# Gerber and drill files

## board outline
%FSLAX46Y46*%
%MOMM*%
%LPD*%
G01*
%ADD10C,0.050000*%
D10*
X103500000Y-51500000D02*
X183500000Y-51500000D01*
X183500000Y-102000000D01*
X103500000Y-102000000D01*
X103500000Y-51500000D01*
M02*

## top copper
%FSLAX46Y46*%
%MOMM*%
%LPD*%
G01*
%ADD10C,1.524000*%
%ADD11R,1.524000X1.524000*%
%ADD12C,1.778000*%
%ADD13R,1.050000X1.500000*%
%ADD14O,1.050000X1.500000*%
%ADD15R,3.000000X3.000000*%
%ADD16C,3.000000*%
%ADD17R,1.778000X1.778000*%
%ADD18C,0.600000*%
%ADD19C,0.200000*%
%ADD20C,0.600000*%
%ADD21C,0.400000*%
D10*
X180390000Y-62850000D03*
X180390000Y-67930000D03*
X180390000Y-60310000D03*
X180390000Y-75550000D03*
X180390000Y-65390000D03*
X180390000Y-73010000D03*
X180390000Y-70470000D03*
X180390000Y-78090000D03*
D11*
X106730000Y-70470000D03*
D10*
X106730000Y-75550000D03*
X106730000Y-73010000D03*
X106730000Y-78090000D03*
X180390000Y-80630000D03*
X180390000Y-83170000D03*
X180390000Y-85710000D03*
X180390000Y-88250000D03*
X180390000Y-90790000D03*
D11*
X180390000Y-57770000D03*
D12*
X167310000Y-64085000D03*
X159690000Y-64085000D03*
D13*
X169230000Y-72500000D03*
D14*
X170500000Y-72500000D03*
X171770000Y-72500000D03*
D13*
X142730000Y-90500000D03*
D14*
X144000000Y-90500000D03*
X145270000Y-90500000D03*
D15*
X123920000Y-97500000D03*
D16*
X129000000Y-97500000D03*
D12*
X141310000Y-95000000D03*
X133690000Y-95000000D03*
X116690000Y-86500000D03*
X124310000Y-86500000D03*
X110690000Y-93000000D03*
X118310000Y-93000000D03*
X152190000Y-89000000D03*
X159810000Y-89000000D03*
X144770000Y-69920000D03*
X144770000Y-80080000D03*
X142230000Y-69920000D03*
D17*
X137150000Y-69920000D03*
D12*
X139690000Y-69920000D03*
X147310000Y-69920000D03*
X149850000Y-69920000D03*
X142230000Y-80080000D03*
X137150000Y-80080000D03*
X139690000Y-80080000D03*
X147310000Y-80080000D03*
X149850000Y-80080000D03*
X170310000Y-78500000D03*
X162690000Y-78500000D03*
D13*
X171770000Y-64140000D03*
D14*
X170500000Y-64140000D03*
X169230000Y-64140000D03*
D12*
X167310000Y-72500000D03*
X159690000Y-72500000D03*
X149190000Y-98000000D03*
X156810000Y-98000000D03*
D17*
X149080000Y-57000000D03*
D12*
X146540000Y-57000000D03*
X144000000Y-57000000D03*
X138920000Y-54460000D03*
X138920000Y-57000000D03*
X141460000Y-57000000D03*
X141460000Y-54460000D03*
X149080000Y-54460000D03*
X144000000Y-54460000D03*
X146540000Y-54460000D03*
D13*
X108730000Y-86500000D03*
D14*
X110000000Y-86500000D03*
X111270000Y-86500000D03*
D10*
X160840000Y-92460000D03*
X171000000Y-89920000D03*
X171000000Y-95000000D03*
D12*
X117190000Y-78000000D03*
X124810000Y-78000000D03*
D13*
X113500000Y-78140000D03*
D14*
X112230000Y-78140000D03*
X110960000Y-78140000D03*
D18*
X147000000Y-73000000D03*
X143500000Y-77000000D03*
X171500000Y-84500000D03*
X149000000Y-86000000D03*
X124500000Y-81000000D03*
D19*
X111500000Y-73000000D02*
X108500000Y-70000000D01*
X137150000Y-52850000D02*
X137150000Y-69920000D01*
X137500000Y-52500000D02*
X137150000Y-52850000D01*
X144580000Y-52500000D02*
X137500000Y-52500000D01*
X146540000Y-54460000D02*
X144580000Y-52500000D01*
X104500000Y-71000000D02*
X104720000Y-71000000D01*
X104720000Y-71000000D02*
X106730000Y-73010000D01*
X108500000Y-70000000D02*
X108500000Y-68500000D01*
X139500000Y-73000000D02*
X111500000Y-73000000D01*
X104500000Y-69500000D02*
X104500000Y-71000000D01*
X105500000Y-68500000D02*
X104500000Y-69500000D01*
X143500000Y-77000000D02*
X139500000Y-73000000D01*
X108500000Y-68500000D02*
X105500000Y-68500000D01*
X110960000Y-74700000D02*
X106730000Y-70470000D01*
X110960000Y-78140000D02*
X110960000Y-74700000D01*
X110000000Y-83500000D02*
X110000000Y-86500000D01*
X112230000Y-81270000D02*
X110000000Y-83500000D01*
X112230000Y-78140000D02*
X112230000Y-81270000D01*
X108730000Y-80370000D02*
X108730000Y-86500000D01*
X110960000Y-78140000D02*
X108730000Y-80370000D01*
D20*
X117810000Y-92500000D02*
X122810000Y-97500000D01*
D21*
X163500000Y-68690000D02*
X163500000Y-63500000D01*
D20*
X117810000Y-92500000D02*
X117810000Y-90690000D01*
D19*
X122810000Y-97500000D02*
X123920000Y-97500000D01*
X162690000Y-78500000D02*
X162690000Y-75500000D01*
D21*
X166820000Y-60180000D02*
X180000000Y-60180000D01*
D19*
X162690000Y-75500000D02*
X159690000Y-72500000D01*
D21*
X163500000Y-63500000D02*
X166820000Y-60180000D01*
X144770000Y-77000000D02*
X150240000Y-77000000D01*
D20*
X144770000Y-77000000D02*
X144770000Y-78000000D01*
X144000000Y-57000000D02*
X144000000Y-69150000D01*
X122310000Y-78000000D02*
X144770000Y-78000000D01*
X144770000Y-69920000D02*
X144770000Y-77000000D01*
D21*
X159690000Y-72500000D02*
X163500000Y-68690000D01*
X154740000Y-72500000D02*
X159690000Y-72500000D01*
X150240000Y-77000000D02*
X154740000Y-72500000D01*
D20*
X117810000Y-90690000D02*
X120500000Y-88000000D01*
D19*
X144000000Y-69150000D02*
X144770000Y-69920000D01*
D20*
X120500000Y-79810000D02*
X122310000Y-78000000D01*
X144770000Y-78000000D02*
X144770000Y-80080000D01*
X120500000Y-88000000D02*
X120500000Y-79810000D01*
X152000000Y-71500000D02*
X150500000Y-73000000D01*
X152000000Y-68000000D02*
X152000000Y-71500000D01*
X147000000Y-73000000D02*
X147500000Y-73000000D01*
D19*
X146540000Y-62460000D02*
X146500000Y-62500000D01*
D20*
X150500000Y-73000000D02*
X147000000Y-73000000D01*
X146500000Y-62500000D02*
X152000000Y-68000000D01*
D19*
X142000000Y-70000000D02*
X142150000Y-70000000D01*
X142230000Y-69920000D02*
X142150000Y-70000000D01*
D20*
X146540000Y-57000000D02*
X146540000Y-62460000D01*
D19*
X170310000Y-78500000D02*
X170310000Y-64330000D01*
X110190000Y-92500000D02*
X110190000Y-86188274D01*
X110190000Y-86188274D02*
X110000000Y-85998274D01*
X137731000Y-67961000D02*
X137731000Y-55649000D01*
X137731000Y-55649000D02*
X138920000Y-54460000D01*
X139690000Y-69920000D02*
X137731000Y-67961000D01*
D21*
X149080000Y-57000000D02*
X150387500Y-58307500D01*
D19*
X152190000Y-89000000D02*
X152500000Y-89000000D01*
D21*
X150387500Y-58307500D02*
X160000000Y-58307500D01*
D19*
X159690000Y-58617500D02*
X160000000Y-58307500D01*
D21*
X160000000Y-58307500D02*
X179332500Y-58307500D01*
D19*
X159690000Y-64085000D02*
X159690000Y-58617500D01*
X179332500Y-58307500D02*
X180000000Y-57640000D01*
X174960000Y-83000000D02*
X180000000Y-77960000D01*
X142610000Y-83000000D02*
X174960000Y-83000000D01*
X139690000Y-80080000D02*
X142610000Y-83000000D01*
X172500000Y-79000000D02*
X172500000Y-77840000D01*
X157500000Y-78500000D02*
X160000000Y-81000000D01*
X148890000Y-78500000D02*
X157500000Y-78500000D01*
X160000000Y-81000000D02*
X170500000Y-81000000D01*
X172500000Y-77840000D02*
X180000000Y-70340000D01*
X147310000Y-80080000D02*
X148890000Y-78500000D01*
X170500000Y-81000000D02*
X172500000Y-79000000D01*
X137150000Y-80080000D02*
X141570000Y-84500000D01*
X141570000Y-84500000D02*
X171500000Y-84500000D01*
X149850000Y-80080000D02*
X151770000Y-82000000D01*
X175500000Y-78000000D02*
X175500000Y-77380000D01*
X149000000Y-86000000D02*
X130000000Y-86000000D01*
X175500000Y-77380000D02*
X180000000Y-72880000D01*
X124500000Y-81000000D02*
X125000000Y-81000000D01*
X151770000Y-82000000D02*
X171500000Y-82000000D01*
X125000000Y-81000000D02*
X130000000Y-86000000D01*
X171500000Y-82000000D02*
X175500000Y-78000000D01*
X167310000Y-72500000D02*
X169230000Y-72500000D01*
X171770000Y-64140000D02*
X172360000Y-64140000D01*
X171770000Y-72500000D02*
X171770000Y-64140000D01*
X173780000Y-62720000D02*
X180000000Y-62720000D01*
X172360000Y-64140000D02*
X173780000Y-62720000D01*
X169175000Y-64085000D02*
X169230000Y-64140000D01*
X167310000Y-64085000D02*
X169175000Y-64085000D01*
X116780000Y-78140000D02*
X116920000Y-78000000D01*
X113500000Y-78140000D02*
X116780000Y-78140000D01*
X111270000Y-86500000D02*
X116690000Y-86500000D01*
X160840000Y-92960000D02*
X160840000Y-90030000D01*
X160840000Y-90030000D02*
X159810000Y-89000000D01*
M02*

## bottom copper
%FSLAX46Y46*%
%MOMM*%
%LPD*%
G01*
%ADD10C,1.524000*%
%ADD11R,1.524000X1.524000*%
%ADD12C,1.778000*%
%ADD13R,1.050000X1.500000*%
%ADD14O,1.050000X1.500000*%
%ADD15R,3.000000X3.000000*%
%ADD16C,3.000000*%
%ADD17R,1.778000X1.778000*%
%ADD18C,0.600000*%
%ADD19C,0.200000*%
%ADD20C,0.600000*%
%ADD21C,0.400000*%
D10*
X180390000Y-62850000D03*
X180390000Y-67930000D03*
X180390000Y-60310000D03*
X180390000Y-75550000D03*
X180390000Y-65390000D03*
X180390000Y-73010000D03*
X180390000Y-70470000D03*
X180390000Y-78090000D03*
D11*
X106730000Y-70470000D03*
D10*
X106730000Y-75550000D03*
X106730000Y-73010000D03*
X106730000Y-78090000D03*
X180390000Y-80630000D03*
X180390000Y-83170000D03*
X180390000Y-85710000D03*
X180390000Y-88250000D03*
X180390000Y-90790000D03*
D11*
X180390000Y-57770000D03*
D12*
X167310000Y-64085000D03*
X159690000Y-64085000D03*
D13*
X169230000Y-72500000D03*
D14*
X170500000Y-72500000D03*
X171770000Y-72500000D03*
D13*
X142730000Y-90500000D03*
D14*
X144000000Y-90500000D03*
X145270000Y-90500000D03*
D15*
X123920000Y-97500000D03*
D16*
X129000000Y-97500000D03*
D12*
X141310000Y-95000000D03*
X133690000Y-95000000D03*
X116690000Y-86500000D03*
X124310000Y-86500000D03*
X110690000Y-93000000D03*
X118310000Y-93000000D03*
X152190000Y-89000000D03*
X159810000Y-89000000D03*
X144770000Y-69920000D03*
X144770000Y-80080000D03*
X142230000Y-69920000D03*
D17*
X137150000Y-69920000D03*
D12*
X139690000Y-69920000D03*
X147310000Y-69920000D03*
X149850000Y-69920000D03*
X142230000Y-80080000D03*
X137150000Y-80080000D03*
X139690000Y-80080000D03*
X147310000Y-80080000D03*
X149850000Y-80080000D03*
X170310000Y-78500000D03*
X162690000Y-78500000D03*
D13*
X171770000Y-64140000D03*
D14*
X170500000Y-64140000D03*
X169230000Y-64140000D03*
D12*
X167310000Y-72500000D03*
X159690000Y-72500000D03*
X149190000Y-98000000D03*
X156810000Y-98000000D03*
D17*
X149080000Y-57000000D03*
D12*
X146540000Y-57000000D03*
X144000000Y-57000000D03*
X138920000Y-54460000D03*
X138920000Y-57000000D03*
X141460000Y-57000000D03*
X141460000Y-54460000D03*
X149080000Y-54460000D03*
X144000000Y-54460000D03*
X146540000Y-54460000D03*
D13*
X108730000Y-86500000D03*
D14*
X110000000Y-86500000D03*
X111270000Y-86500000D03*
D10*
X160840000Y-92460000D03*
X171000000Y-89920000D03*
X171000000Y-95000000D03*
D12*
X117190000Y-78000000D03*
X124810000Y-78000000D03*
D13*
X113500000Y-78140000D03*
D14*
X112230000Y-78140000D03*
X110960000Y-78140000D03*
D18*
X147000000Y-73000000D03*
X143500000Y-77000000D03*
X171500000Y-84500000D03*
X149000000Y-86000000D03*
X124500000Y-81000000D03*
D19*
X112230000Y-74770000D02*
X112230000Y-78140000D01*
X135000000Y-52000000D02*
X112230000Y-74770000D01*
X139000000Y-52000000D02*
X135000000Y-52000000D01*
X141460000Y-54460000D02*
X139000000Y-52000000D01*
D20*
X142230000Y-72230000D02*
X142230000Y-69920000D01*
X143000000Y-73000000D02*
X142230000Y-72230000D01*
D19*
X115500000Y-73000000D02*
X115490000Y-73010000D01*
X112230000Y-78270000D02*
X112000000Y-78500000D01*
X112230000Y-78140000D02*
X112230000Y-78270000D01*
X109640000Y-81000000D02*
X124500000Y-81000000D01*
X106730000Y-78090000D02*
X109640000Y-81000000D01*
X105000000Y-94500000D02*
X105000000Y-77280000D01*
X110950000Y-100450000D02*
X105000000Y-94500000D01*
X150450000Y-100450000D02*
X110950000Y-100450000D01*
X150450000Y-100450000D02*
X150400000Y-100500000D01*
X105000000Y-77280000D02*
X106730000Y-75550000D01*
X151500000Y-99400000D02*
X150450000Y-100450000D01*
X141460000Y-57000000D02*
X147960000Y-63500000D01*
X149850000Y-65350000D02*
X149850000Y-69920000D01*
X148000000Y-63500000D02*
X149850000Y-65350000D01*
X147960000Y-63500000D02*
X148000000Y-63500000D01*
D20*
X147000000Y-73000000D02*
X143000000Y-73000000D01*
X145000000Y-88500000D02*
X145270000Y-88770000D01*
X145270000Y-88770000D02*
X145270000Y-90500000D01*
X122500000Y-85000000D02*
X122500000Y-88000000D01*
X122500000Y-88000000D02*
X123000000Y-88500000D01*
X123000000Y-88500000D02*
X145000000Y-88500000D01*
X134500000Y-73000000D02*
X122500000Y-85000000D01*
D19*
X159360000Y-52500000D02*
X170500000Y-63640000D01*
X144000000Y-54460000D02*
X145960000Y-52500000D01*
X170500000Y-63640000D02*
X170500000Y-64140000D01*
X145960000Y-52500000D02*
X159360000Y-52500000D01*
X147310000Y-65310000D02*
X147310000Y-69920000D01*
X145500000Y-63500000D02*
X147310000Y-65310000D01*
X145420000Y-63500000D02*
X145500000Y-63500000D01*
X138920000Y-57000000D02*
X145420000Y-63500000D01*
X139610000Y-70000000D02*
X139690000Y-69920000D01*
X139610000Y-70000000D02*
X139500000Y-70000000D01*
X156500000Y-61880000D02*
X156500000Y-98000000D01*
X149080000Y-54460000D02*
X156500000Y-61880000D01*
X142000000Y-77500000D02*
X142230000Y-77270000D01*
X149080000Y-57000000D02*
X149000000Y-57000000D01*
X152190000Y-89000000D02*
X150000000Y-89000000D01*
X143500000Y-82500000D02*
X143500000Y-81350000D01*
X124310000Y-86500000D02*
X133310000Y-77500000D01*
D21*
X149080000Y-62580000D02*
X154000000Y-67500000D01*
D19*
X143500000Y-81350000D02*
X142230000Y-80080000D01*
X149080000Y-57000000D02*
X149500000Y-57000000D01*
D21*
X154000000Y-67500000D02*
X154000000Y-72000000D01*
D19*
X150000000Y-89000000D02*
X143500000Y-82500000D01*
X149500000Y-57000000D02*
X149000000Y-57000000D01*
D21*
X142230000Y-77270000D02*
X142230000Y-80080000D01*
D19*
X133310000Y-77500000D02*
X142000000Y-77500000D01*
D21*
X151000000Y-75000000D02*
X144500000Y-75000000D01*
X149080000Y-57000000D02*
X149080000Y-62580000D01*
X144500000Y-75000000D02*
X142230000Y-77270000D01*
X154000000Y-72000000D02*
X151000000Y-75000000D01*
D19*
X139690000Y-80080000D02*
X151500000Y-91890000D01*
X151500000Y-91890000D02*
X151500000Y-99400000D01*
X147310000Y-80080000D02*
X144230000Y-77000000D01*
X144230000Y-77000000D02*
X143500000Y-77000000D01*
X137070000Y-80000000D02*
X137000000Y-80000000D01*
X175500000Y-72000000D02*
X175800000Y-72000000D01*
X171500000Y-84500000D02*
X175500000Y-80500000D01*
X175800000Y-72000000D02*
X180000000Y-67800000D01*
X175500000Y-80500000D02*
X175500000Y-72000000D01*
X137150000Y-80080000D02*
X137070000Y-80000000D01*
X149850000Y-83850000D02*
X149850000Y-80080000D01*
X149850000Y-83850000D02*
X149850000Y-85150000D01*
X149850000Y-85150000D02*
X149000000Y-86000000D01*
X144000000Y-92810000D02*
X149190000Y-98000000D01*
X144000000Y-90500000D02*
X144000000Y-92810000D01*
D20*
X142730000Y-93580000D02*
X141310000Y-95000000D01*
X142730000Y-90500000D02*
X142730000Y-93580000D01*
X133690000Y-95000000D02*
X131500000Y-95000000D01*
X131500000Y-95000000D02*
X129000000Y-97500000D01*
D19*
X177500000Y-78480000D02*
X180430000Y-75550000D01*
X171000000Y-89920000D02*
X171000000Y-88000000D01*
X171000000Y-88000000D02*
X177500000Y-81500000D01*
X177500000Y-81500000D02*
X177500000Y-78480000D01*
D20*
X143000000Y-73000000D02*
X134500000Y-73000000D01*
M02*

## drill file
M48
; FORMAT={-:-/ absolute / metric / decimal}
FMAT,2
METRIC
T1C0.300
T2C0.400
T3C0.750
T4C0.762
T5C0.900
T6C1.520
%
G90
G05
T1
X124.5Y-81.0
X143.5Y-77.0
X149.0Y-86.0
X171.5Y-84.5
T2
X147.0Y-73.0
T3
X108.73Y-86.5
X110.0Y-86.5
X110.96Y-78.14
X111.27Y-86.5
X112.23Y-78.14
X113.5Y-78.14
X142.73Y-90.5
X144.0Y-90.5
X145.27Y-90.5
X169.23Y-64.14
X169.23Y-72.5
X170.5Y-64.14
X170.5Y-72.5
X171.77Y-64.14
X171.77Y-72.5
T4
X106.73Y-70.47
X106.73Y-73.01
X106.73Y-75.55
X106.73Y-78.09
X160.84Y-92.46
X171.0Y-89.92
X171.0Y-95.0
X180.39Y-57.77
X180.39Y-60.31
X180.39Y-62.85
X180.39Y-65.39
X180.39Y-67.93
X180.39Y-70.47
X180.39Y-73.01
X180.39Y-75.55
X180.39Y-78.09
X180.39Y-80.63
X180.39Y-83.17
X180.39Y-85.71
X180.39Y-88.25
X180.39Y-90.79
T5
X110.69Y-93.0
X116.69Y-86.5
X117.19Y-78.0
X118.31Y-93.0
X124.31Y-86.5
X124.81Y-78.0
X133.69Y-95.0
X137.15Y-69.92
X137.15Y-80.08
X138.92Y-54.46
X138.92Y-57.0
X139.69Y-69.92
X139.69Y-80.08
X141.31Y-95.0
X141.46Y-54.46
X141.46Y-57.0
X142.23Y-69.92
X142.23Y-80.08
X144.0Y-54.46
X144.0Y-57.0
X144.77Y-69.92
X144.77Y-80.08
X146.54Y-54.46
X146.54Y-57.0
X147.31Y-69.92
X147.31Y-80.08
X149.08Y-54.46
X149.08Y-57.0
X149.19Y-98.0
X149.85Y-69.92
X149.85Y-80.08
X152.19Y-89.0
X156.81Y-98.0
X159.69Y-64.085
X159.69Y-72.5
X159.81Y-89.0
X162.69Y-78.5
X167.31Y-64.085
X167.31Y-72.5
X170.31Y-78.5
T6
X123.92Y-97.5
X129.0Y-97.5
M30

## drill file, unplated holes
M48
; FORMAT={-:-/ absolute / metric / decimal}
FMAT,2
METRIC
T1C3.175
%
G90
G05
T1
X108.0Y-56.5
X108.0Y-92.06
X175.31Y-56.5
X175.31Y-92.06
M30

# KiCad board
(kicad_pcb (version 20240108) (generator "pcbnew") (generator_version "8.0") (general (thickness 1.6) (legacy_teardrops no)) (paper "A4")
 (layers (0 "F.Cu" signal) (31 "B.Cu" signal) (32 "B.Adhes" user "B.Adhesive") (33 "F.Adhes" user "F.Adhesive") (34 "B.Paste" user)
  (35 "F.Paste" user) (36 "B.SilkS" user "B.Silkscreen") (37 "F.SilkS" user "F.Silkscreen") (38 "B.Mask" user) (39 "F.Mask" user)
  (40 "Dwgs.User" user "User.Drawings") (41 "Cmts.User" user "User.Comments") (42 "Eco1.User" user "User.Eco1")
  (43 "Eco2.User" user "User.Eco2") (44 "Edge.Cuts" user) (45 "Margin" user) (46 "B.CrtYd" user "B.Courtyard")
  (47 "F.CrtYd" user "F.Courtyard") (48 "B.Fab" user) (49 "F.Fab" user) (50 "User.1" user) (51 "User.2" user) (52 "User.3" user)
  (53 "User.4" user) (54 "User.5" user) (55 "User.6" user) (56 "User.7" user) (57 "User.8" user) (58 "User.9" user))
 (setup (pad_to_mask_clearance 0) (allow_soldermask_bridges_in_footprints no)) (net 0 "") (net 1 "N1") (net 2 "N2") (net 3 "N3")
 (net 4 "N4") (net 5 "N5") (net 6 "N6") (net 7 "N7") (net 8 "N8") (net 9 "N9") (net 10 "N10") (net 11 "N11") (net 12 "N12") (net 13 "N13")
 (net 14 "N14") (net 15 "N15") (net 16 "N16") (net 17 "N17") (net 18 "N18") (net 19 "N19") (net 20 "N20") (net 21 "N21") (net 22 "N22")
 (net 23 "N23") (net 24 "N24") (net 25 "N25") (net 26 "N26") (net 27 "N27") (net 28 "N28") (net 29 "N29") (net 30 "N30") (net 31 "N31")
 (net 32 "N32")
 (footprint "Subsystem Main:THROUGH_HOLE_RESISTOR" (layer "F.Cu") (at 163.5 64.085 180)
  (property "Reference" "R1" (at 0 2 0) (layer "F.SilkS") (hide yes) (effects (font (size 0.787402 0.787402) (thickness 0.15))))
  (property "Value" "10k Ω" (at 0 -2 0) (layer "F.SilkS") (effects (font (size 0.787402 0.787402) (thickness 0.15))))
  (pad "P$1" thru_hole circle (at -3.81 0 180) (size 1.778 1.778) (drill 0.9) (layers "*.Cu" "*.Mask") (remove_unused_layers no)
   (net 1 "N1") (solder_mask_margin 0.102))
  (pad "P$2" thru_hole circle (at 3.81 0 180) (size 1.778 1.778) (drill 0.9) (layers "*.Cu" "*.Mask") (remove_unused_layers no) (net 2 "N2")
   (solder_mask_margin 0.102)))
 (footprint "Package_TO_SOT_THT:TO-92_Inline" (layer "F.Cu") (at 169.23 72.5)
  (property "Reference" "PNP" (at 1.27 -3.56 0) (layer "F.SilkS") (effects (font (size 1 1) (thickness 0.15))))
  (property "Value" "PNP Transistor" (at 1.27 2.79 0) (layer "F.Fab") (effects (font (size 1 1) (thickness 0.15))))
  (pad "1" thru_hole rect (at 0 0) (size 1.05 1.5) (drill 0.75) (layers "*.Cu" "*.Mask") (remove_unused_layers no) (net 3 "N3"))
  (pad "2" thru_hole oval (at 1.27 0) (size 1.05 1.5) (drill 0.75) (layers "*.Cu" "*.Mask") (remove_unused_layers no) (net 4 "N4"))
  (pad "3" thru_hole oval (at 2.54 0) (size 1.05 1.5) (drill 0.75) (layers "*.Cu" "*.Mask") (remove_unused_layers no) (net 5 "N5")))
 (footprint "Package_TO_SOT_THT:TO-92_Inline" (layer "F.Cu") (at 142.73 90.5)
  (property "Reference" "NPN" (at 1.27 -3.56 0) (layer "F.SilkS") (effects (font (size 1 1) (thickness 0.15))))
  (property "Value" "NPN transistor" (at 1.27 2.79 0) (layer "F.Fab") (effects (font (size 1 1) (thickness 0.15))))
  (pad "1" thru_hole rect (at 0 0) (size 1.05 1.5) (drill 0.75) (layers "*.Cu" "*.Mask") (remove_unused_layers no) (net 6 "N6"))
  (pad "2" thru_hole oval (at 1.27 0) (size 1.05 1.5) (drill 0.75) (layers "*.Cu" "*.Mask") (remove_unused_layers no) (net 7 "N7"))
  (pad "3" thru_hole oval (at 2.54 0) (size 1.05 1.5) (drill 0.75) (layers "*.Cu" "*.Mask") (remove_unused_layers no) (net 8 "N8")))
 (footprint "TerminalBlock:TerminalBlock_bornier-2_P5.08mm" (layer "F.Cu") (at 123.92 97.5)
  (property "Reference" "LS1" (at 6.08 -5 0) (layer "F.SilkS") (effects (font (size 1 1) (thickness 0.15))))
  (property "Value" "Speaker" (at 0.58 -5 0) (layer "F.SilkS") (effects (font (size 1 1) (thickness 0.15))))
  (pad "1" thru_hole rect (at 0 0) (size 3 3) (drill 1.52) (layers "*.Cu" "*.Mask") (remove_unused_layers no) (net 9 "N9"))
  (pad "2" thru_hole circle (at 5.08 0) (size 3 3) (drill 1.52) (layers "*.Cu" "*.Mask") (remove_unused_layers no) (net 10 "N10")))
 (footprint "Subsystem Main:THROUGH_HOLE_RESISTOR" (layer "F.Cu") (at 137.5 95 180)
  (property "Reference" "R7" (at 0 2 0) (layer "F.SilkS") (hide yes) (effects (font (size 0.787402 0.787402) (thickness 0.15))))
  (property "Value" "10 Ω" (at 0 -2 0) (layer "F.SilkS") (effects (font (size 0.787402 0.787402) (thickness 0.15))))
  (pad "P$1" thru_hole circle (at -3.81 0 180) (size 1.778 1.778) (drill 0.9) (layers "*.Cu" "*.Mask") (remove_unused_layers no)
   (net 6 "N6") (solder_mask_margin 0.102))
  (pad "P$2" thru_hole circle (at 3.81 0 180) (size 1.778 1.778) (drill 0.9) (layers "*.Cu" "*.Mask") (remove_unused_layers no)
   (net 10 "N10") (solder_mask_margin 0.102)))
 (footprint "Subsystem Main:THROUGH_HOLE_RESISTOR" (layer "F.Cu") (at 120.5 86.5)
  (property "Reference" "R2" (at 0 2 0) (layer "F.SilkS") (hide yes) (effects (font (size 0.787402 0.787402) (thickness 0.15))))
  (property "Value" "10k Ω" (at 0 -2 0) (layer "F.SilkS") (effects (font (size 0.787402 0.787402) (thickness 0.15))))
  (pad "P$1" thru_hole circle (at -3.81 0) (size 1.778 1.778) (drill 0.9) (layers "*.Cu" "*.Mask") (remove_unused_layers no) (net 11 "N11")
   (solder_mask_margin 0.102))
  (pad "P$2" thru_hole circle (at 3.81 0) (size 1.778 1.778) (drill 0.9) (layers "*.Cu" "*.Mask") (remove_unused_layers no) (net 2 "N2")
   (solder_mask_margin 0.102)))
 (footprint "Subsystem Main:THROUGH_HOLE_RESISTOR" (layer "F.Cu") (at 114.5 93)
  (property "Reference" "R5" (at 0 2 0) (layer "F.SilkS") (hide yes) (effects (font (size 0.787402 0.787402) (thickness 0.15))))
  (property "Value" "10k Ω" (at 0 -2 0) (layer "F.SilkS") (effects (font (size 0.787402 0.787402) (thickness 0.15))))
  (pad "P$1" thru_hole circle (at -3.81 0) (size 1.778 1.778) (drill 0.9) (layers "*.Cu" "*.Mask") (remove_unused_layers no) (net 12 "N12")
   (solder_mask_margin 0.102))
  (pad "P$2" thru_hole circle (at 3.81 0) (size 1.778 1.778) (drill 0.9) (layers "*.Cu" "*.Mask") (remove_unused_layers no) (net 9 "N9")
   (solder_mask_margin 0.102)))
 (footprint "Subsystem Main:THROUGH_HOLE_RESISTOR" (layer "F.Cu") (at 156 89)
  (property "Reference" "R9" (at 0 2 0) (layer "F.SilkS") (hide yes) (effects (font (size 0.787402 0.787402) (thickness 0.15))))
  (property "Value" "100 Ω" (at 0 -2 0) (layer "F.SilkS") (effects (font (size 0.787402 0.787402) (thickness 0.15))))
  (pad "P$1" thru_hole circle (at -3.81 0) (size 1.778 1.778) (drill 0.9) (layers "*.Cu" "*.Mask") (remove_unused_layers no) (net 2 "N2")
   (solder_mask_margin 0.102))
  (pad "P$2" thru_hole circle (at 3.81 0) (size 1.778 1.778) (drill 0.9) (layers "*.Cu" "*.Mask") (remove_unused_layers no) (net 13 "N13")
   (solder_mask_margin 0.102)))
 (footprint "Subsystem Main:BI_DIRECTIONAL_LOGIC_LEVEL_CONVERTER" (layer "F.Cu") (at 143.5 75)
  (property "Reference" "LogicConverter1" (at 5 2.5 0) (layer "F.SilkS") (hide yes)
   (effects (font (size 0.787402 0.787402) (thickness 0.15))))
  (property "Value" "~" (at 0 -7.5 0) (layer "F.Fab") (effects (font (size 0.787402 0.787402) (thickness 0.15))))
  (pad "GND1" thru_hole circle (at 1.27 -5.08) (size 1.778 1.778) (drill 0.9) (layers "*.Cu" "*.Mask") (remove_unused_layers no)
   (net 9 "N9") (solder_mask_margin 0.102))
  (pad "GND2" thru_hole circle (at 1.27 5.08) (size 1.778 1.778) (drill 0.9) (layers "*.Cu" "*.Mask") (remove_unused_layers no) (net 9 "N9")
   (solder_mask_margin 0.102))
  (pad "HV" thru_hole circle (at -1.27 -5.08) (size 1.778 1.778) (drill 0.9) (layers "*.Cu" "*.Mask") (remove_unused_layers no) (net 8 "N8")
   (solder_mask_margin 0.102))
  (pad "HV1" thru_hole rect (at -6.35 -5.08) (size 1.778 1.778) (drill 0.9) (layers "*.Cu" "*.Mask") (remove_unused_layers no)
   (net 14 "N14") (solder_mask_margin 0.102))
  (pad "HV2" thru_hole circle (at -3.81 -5.08) (size 1.778 1.778) (drill 0.9) (layers "*.Cu" "*.Mask") (remove_unused_layers no)
   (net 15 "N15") (solder_mask_margin 0.102))
  (pad "HV3" thru_hole circle (at 3.81 -5.08) (size 1.778 1.778) (drill 0.9) (layers "*.Cu" "*.Mask") (remove_unused_layers no)
   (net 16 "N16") (solder_mask_margin 0.102))
  (pad "HV4" thru_hole circle (at 6.35 -5.08) (size 1.778 1.778) (drill 0.9) (layers "*.Cu" "*.Mask") (remove_unused_layers no)
   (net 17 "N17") (solder_mask_margin 0.102))
  (pad "LV" thru_hole circle (at -1.27 5.08) (size 1.778 1.778) (drill 0.9) (layers "*.Cu" "*.Mask") (remove_unused_layers no) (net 2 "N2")
   (solder_mask_margin 0.102))
  (pad "LV1" thru_hole circle (at -6.35 5.08) (size 1.778 1.778) (drill 0.9) (layers "*.Cu" "*.Mask") (remove_unused_layers no)
   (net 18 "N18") (solder_mask_margin 0.102))
  (pad "LV2" thru_hole circle (at -3.81 5.08) (size 1.778 1.778) (drill 0.9) (layers "*.Cu" "*.Mask") (remove_unused_layers no)
   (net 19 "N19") (solder_mask_margin 0.102))
  (pad "LV3" thru_hole circle (at 3.81 5.08) (size 1.778 1.778) (drill 0.9) (layers "*.Cu" "*.Mask") (remove_unused_layers no)
   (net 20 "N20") (solder_mask_margin 0.102))
  (pad "LV4" thru_hole circle (at 6.35 5.08) (size 1.778 1.778) (drill 0.9) (layers "*.Cu" "*.Mask") (remove_unused_layers no)
   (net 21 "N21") (solder_mask_margin 0.102)))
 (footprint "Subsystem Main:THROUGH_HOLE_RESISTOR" (layer "F.Cu") (at 166.5 78.5 180)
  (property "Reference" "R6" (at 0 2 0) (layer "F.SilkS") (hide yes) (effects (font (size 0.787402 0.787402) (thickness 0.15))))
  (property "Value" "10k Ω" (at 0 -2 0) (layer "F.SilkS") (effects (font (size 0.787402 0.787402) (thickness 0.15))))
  (pad "P$1" thru_hole circle (at -3.81 0 180) (size 1.778 1.778) (drill 0.9) (layers "*.Cu" "*.Mask") (remove_unused_layers no)
   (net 4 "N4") (solder_mask_margin 0.102))
  (pad "P$2" thru_hole circle (at 3.81 0 180) (size 1.778 1.778) (drill 0.9) (layers "*.Cu" "*.Mask") (remove_unused_layers no) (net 9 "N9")
   (solder_mask_margin 0.102)))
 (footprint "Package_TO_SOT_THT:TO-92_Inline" (layer "F.Cu") (at 171.77 64.14 180)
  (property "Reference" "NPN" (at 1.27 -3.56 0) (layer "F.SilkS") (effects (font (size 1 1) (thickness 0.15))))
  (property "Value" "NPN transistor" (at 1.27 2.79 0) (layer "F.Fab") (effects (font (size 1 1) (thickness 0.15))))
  (pad "1" thru_hole rect (at 0 0 180) (size 1.05 1.5) (drill 0.75) (layers "*.Cu" "*.Mask") (remove_unused_layers no) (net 5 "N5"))
  (pad "2" thru_hole oval (at 1.27 0 180) (size 1.05 1.5) (drill 0.75) (layers "*.Cu" "*.Mask") (remove_unused_layers no) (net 4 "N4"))
  (pad "3" thru_hole oval (at 2.54 0 180) (size 1.05 1.5) (drill 0.75) (layers "*.Cu" "*.Mask") (remove_unused_layers no) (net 1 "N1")))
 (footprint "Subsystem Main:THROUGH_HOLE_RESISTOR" (layer "F.Cu") (at 163.5 72.5 180)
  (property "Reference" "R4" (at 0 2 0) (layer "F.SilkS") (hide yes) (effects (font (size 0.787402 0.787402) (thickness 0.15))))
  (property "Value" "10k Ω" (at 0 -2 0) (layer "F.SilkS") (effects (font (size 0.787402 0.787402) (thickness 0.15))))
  (pad "P$1" thru_hole circle (at -3.81 0 180) (size 1.778 1.778) (drill 0.9) (layers "*.Cu" "*.Mask") (remove_unused_layers no)
   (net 3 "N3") (solder_mask_margin 0.102))
  (pad "P$2" thru_hole circle (at 3.81 0 180) (size 1.778 1.778) (drill 0.9) (layers "*.Cu" "*.Mask") (remove_unused_layers no) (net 9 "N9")
   (solder_mask_margin 0.102)))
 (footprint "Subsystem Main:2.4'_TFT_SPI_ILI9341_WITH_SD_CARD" (layer "F.Cu") (at 142.29 74.28 180)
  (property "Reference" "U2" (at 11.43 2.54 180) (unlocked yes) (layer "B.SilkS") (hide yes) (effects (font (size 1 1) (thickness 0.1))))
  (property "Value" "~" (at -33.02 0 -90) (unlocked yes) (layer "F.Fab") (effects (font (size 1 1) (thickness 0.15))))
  (pad "" np_thru_hole circle (at -33.02 -17.78 180) (size 2.794 2.794) (drill 3.175) (layers "*.Mask"))
  (pad "" np_thru_hole circle (at -33.02 17.78 180) (size 2.794 2.794) (drill 3.175) (layers "*.Mask"))
  (pad "" np_thru_hole circle (at 34.29 -17.78 180) (size 2.794 2.794) (drill 3.175) (layers "*.Mask"))
  (pad "" np_thru_hole circle (at 34.29 17.78 180) (size 2.794 2.794) (drill 3.175) (layers "*.Mask"))
  (pad "CS" thru_hole circle (at -38.1 11.43 180) (size 1.524 1.524) (drill 0.762) (layers "*.Cu" "*.Mask") (remove_unused_layers no)
   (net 5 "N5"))
  (pad "DC" thru_hole circle (at -38.1 6.35 180) (size 1.524 1.524) (drill 0.762) (layers "*.Cu" "*.Mask") (remove_unused_layers no)
   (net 18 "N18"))
  (pad "GND" thru_hole circle (at -38.1 13.97 180) (size 1.524 1.524) (drill 0.762) (layers "*.Cu" "*.Mask") (remove_unused_layers no)
   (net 9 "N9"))
  (pad "LED" thru_hole circle (at -38.1 -1.27 180) (size 1.524 1.524) (drill 0.762) (layers "*.Cu" "*.Mask") (remove_unused_layers no)
   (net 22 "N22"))
  (pad "RESET" thru_hole circle (at -38.1 8.89 180) (size 1.524 1.524) (drill 0.762) (layers "*.Cu" "*.Mask") (remove_unused_layers no)
   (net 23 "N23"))
  (pad "SCK" thru_hole circle (at -38.1 1.27 180) (size 1.524 1.524) (drill 0.762) (layers "*.Cu" "*.Mask") (remove_unused_layers no)
   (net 21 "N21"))
  (pad "SDI(MOSI)" thru_hole circle (at -38.1 3.81 180) (size 1.524 1.524) (drill 0.762) (layers "*.Cu" "*.Mask") (remove_unused_layers no)
   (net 20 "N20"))
  (pad "SDO(MISO)" thru_hole circle (at -38.1 -3.81 180) (size 1.524 1.524) (drill 0.762) (layers "*.Cu" "*.Mask") (remove_unused_layers no)
   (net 19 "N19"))
  (pad "SD_CS" thru_hole rect (at 35.56 3.81 180) (size 1.524 1.524) (drill 0.762) (layers "*.Cu" "*.Mask") (remove_unused_layers no)
   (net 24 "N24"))
  (pad "SD_MISO" thru_hole circle (at 35.56 -1.27 180) (size 1.524 1.524) (drill 0.762) (layers "*.Cu" "*.Mask") (remove_unused_layers no)
   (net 19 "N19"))
  (pad "SD_MOSI" thru_hole circle (at 35.56 1.27 180) (size 1.524 1.524) (drill 0.762) (layers "*.Cu" "*.Mask") (remove_unused_layers no)
   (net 20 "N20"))
  (pad "SD_SCK" thru_hole circle (at 35.56 -3.81 180) (size 1.524 1.524) (drill 0.762) (layers "*.Cu" "*.Mask") (remove_unused_layers no)
   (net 21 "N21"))
  (pad "T_CLK" thru_hole circle (at -38.1 -6.35 180) (size 1.524 1.524) (drill 0.762) (layers "*.Cu" "*.Mask") (remove_unused_layers no)
   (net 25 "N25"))
  (pad "T_CS" thru_hole circle (at -38.1 -8.89 180) (size 1.524 1.524) (drill 0.762) (layers "*.Cu" "*.Mask") (remove_unused_layers no)
   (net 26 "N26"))
  (pad "T_DIN" thru_hole circle (at -38.1 -11.43 180) (size 1.524 1.524) (drill 0.762) (layers "*.Cu" "*.Mask") (remove_unused_layers no)
   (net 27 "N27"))
  (pad "T_DO" thru_hole circle (at -38.1 -13.97 180) (size 1.524 1.524) (drill 0.762) (layers "*.Cu" "*.Mask") (remove_unused_layers no)
   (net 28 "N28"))
  (pad "T_IRQ" thru_hole circle (at -38.1 -16.51 180) (size 1.524 1.524) (drill 0.762) (layers "*.Cu" "*.Mask") (remove_unused_layers no)
   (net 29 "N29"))
  (pad "Vcc" thru_hole rect (at -38.1 16.51 180) (size 1.524 1.524) (drill 0.762) (layers "*.Cu" "*.Mask") (remove_unused_layers no)
   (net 2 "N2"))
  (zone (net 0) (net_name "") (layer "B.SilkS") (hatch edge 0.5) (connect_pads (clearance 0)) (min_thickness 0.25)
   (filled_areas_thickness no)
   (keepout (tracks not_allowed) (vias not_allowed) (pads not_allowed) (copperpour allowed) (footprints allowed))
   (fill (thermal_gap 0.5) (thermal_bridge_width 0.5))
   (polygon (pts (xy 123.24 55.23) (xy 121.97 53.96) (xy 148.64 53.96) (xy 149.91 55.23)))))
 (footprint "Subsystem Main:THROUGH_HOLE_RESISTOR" (layer "F.Cu") (at 153 98)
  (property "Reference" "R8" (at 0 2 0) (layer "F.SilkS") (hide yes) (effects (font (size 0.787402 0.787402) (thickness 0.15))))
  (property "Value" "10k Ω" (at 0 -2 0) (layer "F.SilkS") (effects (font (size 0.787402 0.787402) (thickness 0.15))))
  (pad "P$1" thru_hole circle (at -3.81 0) (size 1.778 1.778) (drill 0.9) (layers "*.Cu" "*.Mask") (remove_unused_layers no) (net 7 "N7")
   (solder_mask_margin 0.102))
  (pad "P$2" thru_hole circle (at 3.81 0) (size 1.778 1.778) (drill 0.9) (layers "*.Cu" "*.Mask") (remove_unused_layers no) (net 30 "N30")
   (solder_mask_margin 0.102)))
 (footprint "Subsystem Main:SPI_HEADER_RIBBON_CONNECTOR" (layer "F.Cu") (at 144 55.73 180)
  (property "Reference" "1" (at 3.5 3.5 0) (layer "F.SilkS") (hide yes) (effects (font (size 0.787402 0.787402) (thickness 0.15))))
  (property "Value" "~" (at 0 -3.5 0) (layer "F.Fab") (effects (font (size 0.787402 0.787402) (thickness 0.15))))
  (pad "3V3" thru_hole rect (at -5.08 -1.27 180) (size 1.778 1.778) (drill 0.9) (layers "*.Cu" "*.Mask") (remove_unused_layers no)
   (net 2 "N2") (solder_mask_margin 0.102))
  (pad "5V" thru_hole circle (at -2.54 -1.27 180) (size 1.778 1.778) (drill 0.9) (layers "*.Cu" "*.Mask") (remove_unused_layers no)
   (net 8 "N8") (solder_mask_margin 0.102))
  (pad "GND" thru_hole circle (at 0 -1.27 180) (size 1.778 1.778) (drill 0.9) (layers "*.Cu" "*.Mask") (remove_unused_layers no)
   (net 9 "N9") (solder_mask_margin 0.102))
  (pad "MISO" thru_hole circle (at 5.08 1.27 180) (size 1.778 1.778) (drill 0.9) (layers "*.Cu" "*.Mask") (remove_unused_layers no)
   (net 15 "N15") (solder_mask_margin 0.102))
  (pad "MOSI" thru_hole circle (at 5.08 -1.27 180) (size 1.778 1.778) (drill 0.9) (layers "*.Cu" "*.Mask") (remove_unused_layers no)
   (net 16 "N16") (solder_mask_margin 0.102))
  (pad "SCK" thru_hole circle (at 2.54 -1.27 180) (size 1.778 1.778) (drill 0.9) (layers "*.Cu" "*.Mask") (remove_unused_layers no)
   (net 17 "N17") (solder_mask_margin 0.102))
  (pad "SD_CS" thru_hole circle (at 2.54 1.27 180) (size 1.778 1.778) (drill 0.9) (layers "*.Cu" "*.Mask") (remove_unused_layers no)
   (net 12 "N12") (solder_mask_margin 0.102))
  (pad "SPKR" thru_hole circle (at -5.08 1.27 180) (size 1.778 1.778) (drill 0.9) (layers "*.Cu" "*.Mask") (remove_unused_layers no)
   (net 30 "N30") (solder_mask_margin 0.102))
  (pad "TFT_CS" thru_hole circle (at 0 1.27 180) (size 1.778 1.778) (drill 0.9) (layers "*.Cu" "*.Mask") (remove_unused_layers no)
   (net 4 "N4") (solder_mask_margin 0.102))
  (pad "TFT_DC" thru_hole circle (at -2.54 1.27 180) (size 1.778 1.778) (drill 0.9) (layers "*.Cu" "*.Mask") (remove_unused_layers no)
   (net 14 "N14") (solder_mask_margin 0.102)))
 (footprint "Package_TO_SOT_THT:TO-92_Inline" (layer "F.Cu") (at 108.73 86.5)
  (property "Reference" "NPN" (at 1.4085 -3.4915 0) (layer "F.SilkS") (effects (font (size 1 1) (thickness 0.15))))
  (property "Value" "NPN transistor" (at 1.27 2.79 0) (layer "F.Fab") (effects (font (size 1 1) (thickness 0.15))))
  (pad "1" thru_hole rect (at 0 0) (size 1.05 1.5) (drill 0.75) (layers "*.Cu" "*.Mask") (remove_unused_layers no) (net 24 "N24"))
  (pad "2" thru_hole oval (at 1.27 0) (size 1.05 1.5) (drill 0.75) (layers "*.Cu" "*.Mask") (remove_unused_layers no) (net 12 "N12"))
  (pad "3" thru_hole oval (at 2.54 0) (size 1.05 1.5) (drill 0.75) (layers "*.Cu" "*.Mask") (remove_unused_layers no) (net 11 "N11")))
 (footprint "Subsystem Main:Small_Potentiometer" (layer "F.Cu") (at 165.92 92.46)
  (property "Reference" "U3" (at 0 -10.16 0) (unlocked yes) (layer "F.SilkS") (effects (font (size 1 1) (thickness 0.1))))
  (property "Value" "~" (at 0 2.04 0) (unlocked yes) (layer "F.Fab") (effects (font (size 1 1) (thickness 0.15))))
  (pad "Vin" thru_hole circle (at -5.08 0) (size 1.524 1.524) (drill 0.762) (layers "*.Cu" "*.Mask") (remove_unused_layers no)
   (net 13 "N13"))
  (pad "Vout1" thru_hole circle (at 5.08 -2.54) (size 1.524 1.524) (drill 0.762) (layers "*.Cu" "*.Mask") (remove_unused_layers no)
   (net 22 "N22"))
  (pad "Vout2" thru_hole circle (at 5.08 2.54) (size 1.524 1.524) (drill 0.762) (layers "*.Cu" "*.Mask") (remove_unused_layers no)
   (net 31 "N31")))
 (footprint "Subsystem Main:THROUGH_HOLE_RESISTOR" (layer "F.Cu") (at 121 78)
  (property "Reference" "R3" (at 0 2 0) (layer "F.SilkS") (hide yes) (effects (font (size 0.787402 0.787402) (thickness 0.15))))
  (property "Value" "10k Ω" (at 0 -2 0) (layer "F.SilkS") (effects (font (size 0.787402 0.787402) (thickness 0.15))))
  (pad "P$1" thru_hole circle (at -3.81 0) (size 1.778 1.778) (drill 0.9) (layers "*.Cu" "*.Mask") (remove_unused_layers no) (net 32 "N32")
   (solder_mask_margin 0.102))
  (pad "P$2" thru_hole circle (at 3.81 0) (size 1.778 1.778) (drill 0.9) (layers "*.Cu" "*.Mask") (remove_unused_layers no) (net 9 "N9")
   (solder_mask_margin 0.102)))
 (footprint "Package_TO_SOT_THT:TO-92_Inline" (layer "F.Cu") (at 113.5 78.14 180)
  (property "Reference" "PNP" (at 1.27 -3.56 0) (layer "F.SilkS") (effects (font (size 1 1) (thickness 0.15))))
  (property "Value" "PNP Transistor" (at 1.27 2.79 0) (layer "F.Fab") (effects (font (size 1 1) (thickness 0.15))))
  (pad "1" thru_hole rect (at 0 0 180) (size 1.05 1.5) (drill 0.75) (layers "*.Cu" "*.Mask") (remove_unused_layers no) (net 32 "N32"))
  (pad "2" thru_hole oval (at 1.27 0 180) (size 1.05 1.5) (drill 0.75) (layers "*.Cu" "*.Mask") (remove_unused_layers no) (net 12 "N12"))
  (pad "3" thru_hole oval (at 2.54 0 180) (size 1.05 1.5) (drill 0.75) (layers "*.Cu" "*.Mask") (remove_unused_layers no) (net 24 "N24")))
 (gr_rect (start 103.5 51.5) (end 183.5 102) (stroke (width 0.05) (type default)) (fill none) (layer "Edge.Cuts"))
 (segment (start 141.46 57) (end 147.96 63.5) (width 0.2) (layer "B.Cu") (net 17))
 (segment (start 149.85 65.35) (end 149.85 69.92) (width 0.2) (layer "B.Cu") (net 17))
 (segment (start 148 63.5) (end 149.85 65.35) (width 0.2) (layer "B.Cu") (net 17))
 (segment (start 147.96 63.5) (end 148 63.5) (width 0.2) (layer "B.Cu") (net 17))
 (segment (start 117.81 92.5) (end 122.81 97.5) (width 0.6) (layer "F.Cu") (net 9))
 (segment (start 163.5 68.69) (end 163.5 63.5) (width 0.4) (layer "F.Cu") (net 9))
 (segment (start 117.81 92.5) (end 117.81 90.69) (width 0.6) (layer "F.Cu") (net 9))
 (segment (start 122.81 97.5) (end 123.92 97.5) (width 0.2) (layer "F.Cu") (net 9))
 (segment (start 162.69 78.5) (end 162.69 75.5) (width 0.2) (layer "F.Cu") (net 9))
 (segment (start 166.82 60.18) (end 180 60.18) (width 0.4) (layer "F.Cu") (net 9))
 (segment (start 162.69 75.5) (end 159.69 72.5) (width 0.2) (layer "F.Cu") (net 9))
 (segment (start 163.5 63.5) (end 166.82 60.18) (width 0.4) (layer "F.Cu") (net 9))
 (segment (start 144.77 77) (end 150.24 77) (width 0.4) (layer "F.Cu") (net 9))
 (segment (start 144.77 77) (end 144.77 78) (width 0.6) (layer "F.Cu") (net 9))
 (segment (start 144 57) (end 144 69.15) (width 0.6) (layer "F.Cu") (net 9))
 (segment (start 122.31 78) (end 144.77 78) (width 0.6) (layer "F.Cu") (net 9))
 (segment (start 144.77 69.92) (end 144.77 77) (width 0.6) (layer "F.Cu") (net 9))
 (segment (start 159.69 72.5) (end 163.5 68.69) (width 0.4) (layer "F.Cu") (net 9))
 (segment (start 154.74 72.5) (end 159.69 72.5) (width 0.4) (layer "F.Cu") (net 9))
 (segment (start 150.24 77) (end 154.74 72.5) (width 0.4) (layer "F.Cu") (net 9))
 (segment (start 117.81 90.69) (end 120.5 88) (width 0.6) (layer "F.Cu") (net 9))
 (segment (start 144 69.15) (end 144.77 69.92) (width 0.2) (layer "F.Cu") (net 9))
 (segment (start 120.5 79.81) (end 122.31 78) (width 0.6) (layer "F.Cu") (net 9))
 (segment (start 144.77 78) (end 144.77 80.08) (width 0.6) (layer "F.Cu") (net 9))
 (segment (start 120.5 88) (end 120.5 79.81) (width 0.6) (layer "F.Cu") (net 9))
 (segment (start 152 71.5) (end 150.5 73) (width 0.6) (layer "F.Cu") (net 8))
 (segment (start 152 68) (end 152 71.5) (width 0.6) (layer "F.Cu") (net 8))
 (segment (start 147 73) (end 147.5 73) (width 0.6) (layer "F.Cu") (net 8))
 (segment (start 146.54 62.46) (end 146.5 62.5) (width 0.2) (layer "F.Cu") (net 8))
 (segment (start 150.5 73) (end 147 73) (width 0.6) (layer "F.Cu") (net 8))
 (segment (start 146.5 62.5) (end 152 68) (width 0.6) (layer "F.Cu") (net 8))
 (segment (start 142 70) (end 142.15 70) (width 0.2) (layer "F.Cu") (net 8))
 (segment (start 142.23 69.92) (end 142.15 70) (width 0.2) (layer "F.Cu") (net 8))
 (segment (start 146.54 57) (end 146.54 62.46) (width 0.6) (layer "F.Cu") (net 8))
 (via (at 147 73) (size 0.6) (drill 0.4) (layers "F.Cu" "B.Cu") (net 8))
 (segment (start 147 73) (end 143 73) (width 0.6) (layer "B.Cu") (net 8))
 (segment (start 145 88.5) (end 145.27 88.77) (width 0.6) (layer "B.Cu") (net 8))
 (segment (start 143 73) (end 142.23 72.23) (width 0.6) (layer "B.Cu") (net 8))
 (segment (start 145.27 88.77) (end 145.27 90.5) (width 0.6) (layer "B.Cu") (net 8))
 (segment (start 122.5 85) (end 122.5 88) (width 0.6) (layer "B.Cu") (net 8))
 (segment (start 143 73) (end 134.5 73) (width 0.6) (layer "B.Cu") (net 8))
 (segment (start 122.5 88) (end 123 88.5) (width 0.6) (layer "B.Cu") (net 8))
 (segment (start 123 88.5) (end 145 88.5) (width 0.6) (layer "B.Cu") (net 8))
 (segment (start 134.5 73) (end 122.5 85) (width 0.6) (layer "B.Cu") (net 8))
 (segment (start 142.23 72.23) (end 142.23 69.92) (width 0.6) (layer "B.Cu") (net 8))
 (segment (start 170.31 78.5) (end 170.31 64.33) (width 0.2) (layer "F.Cu") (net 4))
 (segment (start 159.36 52.5) (end 170.5 63.64) (width 0.2) (layer "B.Cu") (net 4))
 (segment (start 144 54.46) (end 145.96 52.5) (width 0.2) (layer "B.Cu") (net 4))
 (segment (start 170.5 63.64) (end 170.5 64.14) (width 0.2) (layer "B.Cu") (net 4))
 (segment (start 145.96 52.5) (end 159.36 52.5) (width 0.2) (layer "B.Cu") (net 4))
 (segment (start 147.31 65.31) (end 147.31 69.92) (width 0.2) (layer "B.Cu") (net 16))
 (segment (start 145.5 63.5) (end 147.31 65.31) (width 0.2) (layer "B.Cu") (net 16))
 (segment (start 145.42 63.5) (end 145.5 63.5) (width 0.2) (layer "B.Cu") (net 16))
 (segment (start 138.92 57) (end 145.42 63.5) (width 0.2) (layer "B.Cu") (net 16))
 (segment (start 110.19 92.5) (end 110.19 86.188274) (width 0.2) (layer "F.Cu") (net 12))
 (segment (start 110.19 86.188274) (end 110 85.998274) (width 0.2) (layer "F.Cu") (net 12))
 (segment (start 112.23 81.27) (end 110 83.5) (width 0.2) (layer "F.Cu") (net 12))
 (segment (start 112.23 78.14) (end 112.23 81.27) (width 0.2) (layer "F.Cu") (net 12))
 (segment (start 110 83.5) (end 110 86.5) (width 0.2) (layer "F.Cu") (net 12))
 (segment (start 135 52) (end 112.23 74.77) (width 0.2) (layer "B.Cu") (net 12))
 (segment (start 141.46 54.46) (end 139 52) (width 0.2) (layer "B.Cu") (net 12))
 (segment (start 139 52) (end 135 52) (width 0.2) (layer "B.Cu") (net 12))
 (segment (start 112.23 74.77) (end 112.23 78.14) (width 0.2) (layer "B.Cu") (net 12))
 (segment (start 112.23 78.27) (end 112 78.5) (width 0.2) (layer "B.Cu") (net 12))
 (segment (start 112.23 78.14) (end 112.23 78.27) (width 0.2) (layer "B.Cu") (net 12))
 (segment (start 137.731 67.961) (end 137.731 55.649) (width 0.2) (layer "F.Cu") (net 15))
 (segment (start 137.731 55.649) (end 138.92 54.46) (width 0.2) (layer "F.Cu") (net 15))
 (segment (start 139.69 69.92) (end 137.731 67.961) (width 0.2) (layer "F.Cu") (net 15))
 (segment (start 139.61 70) (end 139.69 69.92) (width 0.2) (layer "B.Cu") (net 15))
 (segment (start 139.61 70) (end 139.5 70) (width 0.2) (layer "B.Cu") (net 15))
 (segment (start 156.5 61.88) (end 156.5 98) (width 0.2) (layer "B.Cu") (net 30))
 (segment (start 149.08 54.46) (end 156.5 61.88) (width 0.2) (layer "B.Cu") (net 30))
 (segment (start 137.15 52.85) (end 137.15 69.92) (width 0.2) (layer "F.Cu") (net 14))
 (segment (start 144.58 52.5) (end 137.5 52.5) (width 0.2) (layer "F.Cu") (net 14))
 (segment (start 137.5 52.5) (end 137.15 52.85) (width 0.2) (layer "F.Cu") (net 14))
 (segment (start 146.54 54.46) (end 144.58 52.5) (width 0.2) (layer "F.Cu") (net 14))
 (segment (start 149.08 57) (end 150.3875 58.3075) (width 0.4) (layer "F.Cu") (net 2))
 (segment (start 152.19 89) (end 152.5 89) (width 0.2) (layer "F.Cu") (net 2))
 (segment (start 150.3875 58.3075) (end 160 58.3075) (width 0.4) (layer "F.Cu") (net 2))
 (segment (start 159.69 58.6175) (end 160 58.3075) (width 0.2) (layer "F.Cu") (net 2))
 (segment (start 160 58.3075) (end 179.3325 58.3075) (width 0.4) (layer "F.Cu") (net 2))
 (segment (start 159.69 64.085) (end 159.69 58.6175) (width 0.2) (layer "F.Cu") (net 2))
 (segment (start 179.3325 58.3075) (end 180 57.64) (width 0.2) (layer "F.Cu") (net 2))
 (segment (start 142 77.5) (end 142.23 77.27) (width 0.2) (layer "B.Cu") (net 2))
 (segment (start 149.08 57) (end 149 57) (width 0.2) (layer "B.Cu") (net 2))
 (segment (start 152.19 89) (end 150 89) (width 0.2) (layer "B.Cu") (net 2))
 (segment (start 143.5 82.5) (end 143.5 81.35) (width 0.2) (layer "B.Cu") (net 2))
 (segment (start 124.31 86.5) (end 133.31 77.5) (width 0.2) (layer "B.Cu") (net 2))
 (segment (start 149.08 62.58) (end 154 67.5) (width 0.4) (layer "B.Cu") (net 2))
 (segment (start 143.5 81.35) (end 142.23 80.08) (width 0.2) (layer "B.Cu") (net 2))
 (segment (start 149.08 57) (end 149.5 57) (width 0.2) (layer "B.Cu") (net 2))
 (segment (start 154 67.5) (end 154 72) (width 0.4) (layer "B.Cu") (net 2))
 (segment (start 150 89) (end 143.5 82.5) (width 0.2) (layer "B.Cu") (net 2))
 (segment (start 149.5 57) (end 149 57) (width 0.2) (layer "B.Cu") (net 2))
 (segment (start 142.23 77.27) (end 142.23 80.08) (width 0.4) (layer "B.Cu") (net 2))
 (segment (start 133.31 77.5) (end 142 77.5) (width 0.2) (layer "B.Cu") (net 2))
 (segment (start 151 75) (end 144.5 75) (width 0.4) (layer "B.Cu") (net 2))
 (segment (start 149.08 57) (end 149.08 62.58) (width 0.4) (layer "B.Cu") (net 2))
 (segment (start 144.5 75) (end 142.23 77.27) (width 0.4) (layer "B.Cu") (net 2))
 (segment (start 154 72) (end 151 75) (width 0.4) (layer "B.Cu") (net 2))
 (segment (start 174.96 83) (end 180 77.96) (width 0.2) (layer "F.Cu") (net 19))
 (segment (start 142.61 83) (end 174.96 83) (width 0.2) (layer "F.Cu") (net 19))
 (segment (start 139.69 80.08) (end 142.61 83) (width 0.2) (layer "F.Cu") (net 19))
 (segment (start 150.45 100.45) (end 110.95 100.45) (width 0.2) (layer "B.Cu") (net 19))
 (segment (start 151.5 99.4) (end 150.45 100.45) (width 0.2) (layer "B.Cu") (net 19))
 (segment (start 139.69 80.08) (end 151.5 91.89) (width 0.2) (layer "B.Cu") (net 19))
 (segment (start 151.5 91.89) (end 151.5 99.4) (width 0.2) (layer "B.Cu") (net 19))
 (segment (start 105 77.28) (end 106.73 75.55) (width 0.2) (layer "B.Cu") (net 19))
 (segment (start 150.45 100.45) (end 150.4 100.5) (width 0.2) (layer "B.Cu") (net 19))
 (segment (start 110.95 100.45) (end 105 94.5) (width 0.2) (layer "B.Cu") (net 19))
 (segment (start 105 94.5) (end 105 77.28) (width 0.2) (layer "B.Cu") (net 19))
 (segment (start 108.5 68.5) (end 105.5 68.5) (width 0.2) (layer "F.Cu") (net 20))
 (segment (start 104.5 71) (end 104.72 71) (width 0.2) (layer "F.Cu") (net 20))
 (segment (start 172.5 79) (end 172.5 77.84) (width 0.2) (layer "F.Cu") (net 20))
 (segment (start 104.72 71) (end 106.73 73.01) (width 0.2) (layer "F.Cu") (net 20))
 (segment (start 108.5 70) (end 108.5 68.5) (width 0.2) (layer "F.Cu") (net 20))
 (segment (start 157.5 78.5) (end 160 81) (width 0.2) (layer "F.Cu") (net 20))
 (segment (start 148.89 78.5) (end 157.5 78.5) (width 0.2) (layer "F.Cu") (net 20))
 (segment (start 104.5 69.5) (end 104.5 71) (width 0.2) (layer "F.Cu") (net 20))
 (segment (start 160 81) (end 170.5 81) (width 0.2) (layer "F.Cu") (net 20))
 (segment (start 172.5 77.84) (end 180 70.34) (width 0.2) (layer "F.Cu") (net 20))
 (segment (start 147.31 80.08) (end 148.89 78.5) (width 0.2) (layer "F.Cu") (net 20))
 (segment (start 105.5 68.5) (end 104.5 69.5) (width 0.2) (layer "F.Cu") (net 20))
 (segment (start 139.5 73) (end 111.5 73) (width 0.2) (layer "F.Cu") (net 20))
 (segment (start 143.5 77) (end 139.5 73) (width 0.2) (layer "F.Cu") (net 20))
 (segment (start 170.5 81) (end 172.5 79) (width 0.2) (layer "F.Cu") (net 20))
 (segment (start 111.5 73) (end 108.5 70) (width 0.2) (layer "F.Cu") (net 20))
 (via (at 143.5 77) (size 0.6) (drill 0.3) (layers "F.Cu" "B.Cu") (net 20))
 (segment (start 147.31 80.08) (end 144.23 77) (width 0.2) (layer "B.Cu") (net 20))
 (segment (start 115.5 73) (end 115.49 73.01) (width 0.2) (layer "B.Cu") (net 20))
 (segment (start 144.23 77) (end 143.5 77) (width 0.2) (layer "B.Cu") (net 20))
 (segment (start 137.15 80.08) (end 141.57 84.5) (width 0.2) (layer "F.Cu") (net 18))
 (segment (start 141.57 84.5) (end 171.5 84.5) (width 0.2) (layer "F.Cu") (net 18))
 (via (at 171.5 84.5) (size 0.6) (drill 0.3) (layers "F.Cu" "B.Cu") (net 18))
 (segment (start 137.07 80) (end 137 80) (width 0.2) (layer "B.Cu") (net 18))
 (segment (start 175.5 72) (end 175.8 72) (width 0.2) (layer "B.Cu") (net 18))
 (segment (start 171.5 84.5) (end 175.5 80.5) (width 0.2) (layer "B.Cu") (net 18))
 (segment (start 175.8 72) (end 180 67.8) (width 0.2) (layer "B.Cu") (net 18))
 (segment (start 175.5 80.5) (end 175.5 72) (width 0.2) (layer "B.Cu") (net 18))
 (segment (start 137.15 80.08) (end 137.07 80) (width 0.2) (layer "B.Cu") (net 18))
 (segment (start 149.85 80.08) (end 151.77 82) (width 0.2) (layer "F.Cu") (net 21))
 (segment (start 175.5 78) (end 175.5 77.38) (width 0.2) (layer "F.Cu") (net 21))
 (segment (start 149 86) (end 130 86) (width 0.2) (layer "F.Cu") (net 21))
 (segment (start 175.5 77.38) (end 180 72.88) (width 0.2) (layer "F.Cu") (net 21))
 (segment (start 124.5 81) (end 125 81) (width 0.2) (layer "F.Cu") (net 21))
 (segment (start 151.77 82) (end 171.5 82) (width 0.2) (layer "F.Cu") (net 21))
 (segment (start 125 81) (end 130 86) (width 0.2) (layer "F.Cu") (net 21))
 (segment (start 171.5 82) (end 175.5 78) (width 0.2) (layer "F.Cu") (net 21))
 (via (at 149 86) (size 0.6) (drill 0.3) (layers "F.Cu" "B.Cu") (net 21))
 (via (at 124.5 81) (size 0.6) (drill 0.3) (layers "F.Cu" "B.Cu") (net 21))
 (segment (start 109.64 81) (end 124.5 81) (width 0.2) (layer "B.Cu") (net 21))
 (segment (start 149.85 83.85) (end 149.85 80.08) (width 0.2) (layer "B.Cu") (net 21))
 (segment (start 106.73 78.09) (end 109.64 81) (width 0.2) (layer "B.Cu") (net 21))
 (segment (start 149.85 83.85) (end 149.85 85.15) (width 0.2) (layer "B.Cu") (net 21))
 (segment (start 149.85 85.15) (end 149 86) (width 0.2) (layer "B.Cu") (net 21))
 (segment (start 167.31 72.5) (end 169.23 72.5) (width 0.2) (layer "F.Cu") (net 3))
 (segment (start 171.77 64.14) (end 172.36 64.14) (width 0.2) (layer "F.Cu") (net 5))
 (segment (start 171.77 72.5) (end 171.77 64.14) (width 0.2) (layer "F.Cu") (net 5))
 (segment (start 173.78 62.72) (end 180 62.72) (width 0.2) (layer "F.Cu") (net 5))
 (segment (start 172.36 64.14) (end 173.78 62.72) (width 0.2) (layer "F.Cu") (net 5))
 (segment (start 169.175 64.085) (end 169.23 64.14) (width 0.2) (layer "F.Cu") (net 1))
 (segment (start 167.31 64.085) (end 169.175 64.085) (width 0.2) (layer "F.Cu") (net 1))
 (segment (start 110.96 74.7) (end 106.73 70.47) (width 0.2) (layer "F.Cu") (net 24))
 (segment (start 110.96 78.14) (end 108.73 80.37) (width 0.2) (layer "F.Cu") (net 24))
 (segment (start 110.96 78.14) (end 110.96 74.7) (width 0.2) (layer "F.Cu") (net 24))
 (segment (start 108.73 80.37) (end 108.73 86.5) (width 0.2) (layer "F.Cu") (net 24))
 (segment (start 116.78 78.14) (end 116.92 78) (width 0.2) (layer "F.Cu") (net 32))
 (segment (start 113.5 78.14) (end 116.78 78.14) (width 0.2) (layer "F.Cu") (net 32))
 (segment (start 111.27 86.5) (end 116.69 86.5) (width 0.2) (layer "F.Cu") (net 11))
 (segment (start 160.84 92.96) (end 160.84 90.03) (width 0.2) (layer "F.Cu") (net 13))
 (segment (start 160.84 90.03) (end 159.81 89) (width 0.2) (layer "F.Cu") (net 13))
 (segment (start 144 92.81) (end 149.19 98) (width 0.2) (layer "B.Cu") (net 7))
 (segment (start 144 90.5) (end 144 92.81) (width 0.2) (layer "B.Cu") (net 7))
 (segment (start 142.73 93.58) (end 141.31 95) (width 0.6) (layer "B.Cu") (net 6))
 (segment (start 142.73 90.5) (end 142.73 93.58) (width 0.6) (layer "B.Cu") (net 6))
 (segment (start 133.69 95) (end 131.5 95) (width 0.6) (layer "B.Cu") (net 10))
 (segment (start 131.5 95) (end 129 97.5) (width 0.6) (layer "B.Cu") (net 10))
 (segment (start 177.5 78.48) (end 180.43 75.55) (width 0.2) (layer "B.Cu") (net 22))
 (segment (start 171 89.92) (end 171 88) (width 0.2) (layer "B.Cu") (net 22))
 (segment (start 171 88) (end 177.5 81.5) (width 0.2) (layer "B.Cu") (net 22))
 (segment (start 177.5 81.5) (end 177.5 78.48) (width 0.2) (layer "B.Cu") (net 22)))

